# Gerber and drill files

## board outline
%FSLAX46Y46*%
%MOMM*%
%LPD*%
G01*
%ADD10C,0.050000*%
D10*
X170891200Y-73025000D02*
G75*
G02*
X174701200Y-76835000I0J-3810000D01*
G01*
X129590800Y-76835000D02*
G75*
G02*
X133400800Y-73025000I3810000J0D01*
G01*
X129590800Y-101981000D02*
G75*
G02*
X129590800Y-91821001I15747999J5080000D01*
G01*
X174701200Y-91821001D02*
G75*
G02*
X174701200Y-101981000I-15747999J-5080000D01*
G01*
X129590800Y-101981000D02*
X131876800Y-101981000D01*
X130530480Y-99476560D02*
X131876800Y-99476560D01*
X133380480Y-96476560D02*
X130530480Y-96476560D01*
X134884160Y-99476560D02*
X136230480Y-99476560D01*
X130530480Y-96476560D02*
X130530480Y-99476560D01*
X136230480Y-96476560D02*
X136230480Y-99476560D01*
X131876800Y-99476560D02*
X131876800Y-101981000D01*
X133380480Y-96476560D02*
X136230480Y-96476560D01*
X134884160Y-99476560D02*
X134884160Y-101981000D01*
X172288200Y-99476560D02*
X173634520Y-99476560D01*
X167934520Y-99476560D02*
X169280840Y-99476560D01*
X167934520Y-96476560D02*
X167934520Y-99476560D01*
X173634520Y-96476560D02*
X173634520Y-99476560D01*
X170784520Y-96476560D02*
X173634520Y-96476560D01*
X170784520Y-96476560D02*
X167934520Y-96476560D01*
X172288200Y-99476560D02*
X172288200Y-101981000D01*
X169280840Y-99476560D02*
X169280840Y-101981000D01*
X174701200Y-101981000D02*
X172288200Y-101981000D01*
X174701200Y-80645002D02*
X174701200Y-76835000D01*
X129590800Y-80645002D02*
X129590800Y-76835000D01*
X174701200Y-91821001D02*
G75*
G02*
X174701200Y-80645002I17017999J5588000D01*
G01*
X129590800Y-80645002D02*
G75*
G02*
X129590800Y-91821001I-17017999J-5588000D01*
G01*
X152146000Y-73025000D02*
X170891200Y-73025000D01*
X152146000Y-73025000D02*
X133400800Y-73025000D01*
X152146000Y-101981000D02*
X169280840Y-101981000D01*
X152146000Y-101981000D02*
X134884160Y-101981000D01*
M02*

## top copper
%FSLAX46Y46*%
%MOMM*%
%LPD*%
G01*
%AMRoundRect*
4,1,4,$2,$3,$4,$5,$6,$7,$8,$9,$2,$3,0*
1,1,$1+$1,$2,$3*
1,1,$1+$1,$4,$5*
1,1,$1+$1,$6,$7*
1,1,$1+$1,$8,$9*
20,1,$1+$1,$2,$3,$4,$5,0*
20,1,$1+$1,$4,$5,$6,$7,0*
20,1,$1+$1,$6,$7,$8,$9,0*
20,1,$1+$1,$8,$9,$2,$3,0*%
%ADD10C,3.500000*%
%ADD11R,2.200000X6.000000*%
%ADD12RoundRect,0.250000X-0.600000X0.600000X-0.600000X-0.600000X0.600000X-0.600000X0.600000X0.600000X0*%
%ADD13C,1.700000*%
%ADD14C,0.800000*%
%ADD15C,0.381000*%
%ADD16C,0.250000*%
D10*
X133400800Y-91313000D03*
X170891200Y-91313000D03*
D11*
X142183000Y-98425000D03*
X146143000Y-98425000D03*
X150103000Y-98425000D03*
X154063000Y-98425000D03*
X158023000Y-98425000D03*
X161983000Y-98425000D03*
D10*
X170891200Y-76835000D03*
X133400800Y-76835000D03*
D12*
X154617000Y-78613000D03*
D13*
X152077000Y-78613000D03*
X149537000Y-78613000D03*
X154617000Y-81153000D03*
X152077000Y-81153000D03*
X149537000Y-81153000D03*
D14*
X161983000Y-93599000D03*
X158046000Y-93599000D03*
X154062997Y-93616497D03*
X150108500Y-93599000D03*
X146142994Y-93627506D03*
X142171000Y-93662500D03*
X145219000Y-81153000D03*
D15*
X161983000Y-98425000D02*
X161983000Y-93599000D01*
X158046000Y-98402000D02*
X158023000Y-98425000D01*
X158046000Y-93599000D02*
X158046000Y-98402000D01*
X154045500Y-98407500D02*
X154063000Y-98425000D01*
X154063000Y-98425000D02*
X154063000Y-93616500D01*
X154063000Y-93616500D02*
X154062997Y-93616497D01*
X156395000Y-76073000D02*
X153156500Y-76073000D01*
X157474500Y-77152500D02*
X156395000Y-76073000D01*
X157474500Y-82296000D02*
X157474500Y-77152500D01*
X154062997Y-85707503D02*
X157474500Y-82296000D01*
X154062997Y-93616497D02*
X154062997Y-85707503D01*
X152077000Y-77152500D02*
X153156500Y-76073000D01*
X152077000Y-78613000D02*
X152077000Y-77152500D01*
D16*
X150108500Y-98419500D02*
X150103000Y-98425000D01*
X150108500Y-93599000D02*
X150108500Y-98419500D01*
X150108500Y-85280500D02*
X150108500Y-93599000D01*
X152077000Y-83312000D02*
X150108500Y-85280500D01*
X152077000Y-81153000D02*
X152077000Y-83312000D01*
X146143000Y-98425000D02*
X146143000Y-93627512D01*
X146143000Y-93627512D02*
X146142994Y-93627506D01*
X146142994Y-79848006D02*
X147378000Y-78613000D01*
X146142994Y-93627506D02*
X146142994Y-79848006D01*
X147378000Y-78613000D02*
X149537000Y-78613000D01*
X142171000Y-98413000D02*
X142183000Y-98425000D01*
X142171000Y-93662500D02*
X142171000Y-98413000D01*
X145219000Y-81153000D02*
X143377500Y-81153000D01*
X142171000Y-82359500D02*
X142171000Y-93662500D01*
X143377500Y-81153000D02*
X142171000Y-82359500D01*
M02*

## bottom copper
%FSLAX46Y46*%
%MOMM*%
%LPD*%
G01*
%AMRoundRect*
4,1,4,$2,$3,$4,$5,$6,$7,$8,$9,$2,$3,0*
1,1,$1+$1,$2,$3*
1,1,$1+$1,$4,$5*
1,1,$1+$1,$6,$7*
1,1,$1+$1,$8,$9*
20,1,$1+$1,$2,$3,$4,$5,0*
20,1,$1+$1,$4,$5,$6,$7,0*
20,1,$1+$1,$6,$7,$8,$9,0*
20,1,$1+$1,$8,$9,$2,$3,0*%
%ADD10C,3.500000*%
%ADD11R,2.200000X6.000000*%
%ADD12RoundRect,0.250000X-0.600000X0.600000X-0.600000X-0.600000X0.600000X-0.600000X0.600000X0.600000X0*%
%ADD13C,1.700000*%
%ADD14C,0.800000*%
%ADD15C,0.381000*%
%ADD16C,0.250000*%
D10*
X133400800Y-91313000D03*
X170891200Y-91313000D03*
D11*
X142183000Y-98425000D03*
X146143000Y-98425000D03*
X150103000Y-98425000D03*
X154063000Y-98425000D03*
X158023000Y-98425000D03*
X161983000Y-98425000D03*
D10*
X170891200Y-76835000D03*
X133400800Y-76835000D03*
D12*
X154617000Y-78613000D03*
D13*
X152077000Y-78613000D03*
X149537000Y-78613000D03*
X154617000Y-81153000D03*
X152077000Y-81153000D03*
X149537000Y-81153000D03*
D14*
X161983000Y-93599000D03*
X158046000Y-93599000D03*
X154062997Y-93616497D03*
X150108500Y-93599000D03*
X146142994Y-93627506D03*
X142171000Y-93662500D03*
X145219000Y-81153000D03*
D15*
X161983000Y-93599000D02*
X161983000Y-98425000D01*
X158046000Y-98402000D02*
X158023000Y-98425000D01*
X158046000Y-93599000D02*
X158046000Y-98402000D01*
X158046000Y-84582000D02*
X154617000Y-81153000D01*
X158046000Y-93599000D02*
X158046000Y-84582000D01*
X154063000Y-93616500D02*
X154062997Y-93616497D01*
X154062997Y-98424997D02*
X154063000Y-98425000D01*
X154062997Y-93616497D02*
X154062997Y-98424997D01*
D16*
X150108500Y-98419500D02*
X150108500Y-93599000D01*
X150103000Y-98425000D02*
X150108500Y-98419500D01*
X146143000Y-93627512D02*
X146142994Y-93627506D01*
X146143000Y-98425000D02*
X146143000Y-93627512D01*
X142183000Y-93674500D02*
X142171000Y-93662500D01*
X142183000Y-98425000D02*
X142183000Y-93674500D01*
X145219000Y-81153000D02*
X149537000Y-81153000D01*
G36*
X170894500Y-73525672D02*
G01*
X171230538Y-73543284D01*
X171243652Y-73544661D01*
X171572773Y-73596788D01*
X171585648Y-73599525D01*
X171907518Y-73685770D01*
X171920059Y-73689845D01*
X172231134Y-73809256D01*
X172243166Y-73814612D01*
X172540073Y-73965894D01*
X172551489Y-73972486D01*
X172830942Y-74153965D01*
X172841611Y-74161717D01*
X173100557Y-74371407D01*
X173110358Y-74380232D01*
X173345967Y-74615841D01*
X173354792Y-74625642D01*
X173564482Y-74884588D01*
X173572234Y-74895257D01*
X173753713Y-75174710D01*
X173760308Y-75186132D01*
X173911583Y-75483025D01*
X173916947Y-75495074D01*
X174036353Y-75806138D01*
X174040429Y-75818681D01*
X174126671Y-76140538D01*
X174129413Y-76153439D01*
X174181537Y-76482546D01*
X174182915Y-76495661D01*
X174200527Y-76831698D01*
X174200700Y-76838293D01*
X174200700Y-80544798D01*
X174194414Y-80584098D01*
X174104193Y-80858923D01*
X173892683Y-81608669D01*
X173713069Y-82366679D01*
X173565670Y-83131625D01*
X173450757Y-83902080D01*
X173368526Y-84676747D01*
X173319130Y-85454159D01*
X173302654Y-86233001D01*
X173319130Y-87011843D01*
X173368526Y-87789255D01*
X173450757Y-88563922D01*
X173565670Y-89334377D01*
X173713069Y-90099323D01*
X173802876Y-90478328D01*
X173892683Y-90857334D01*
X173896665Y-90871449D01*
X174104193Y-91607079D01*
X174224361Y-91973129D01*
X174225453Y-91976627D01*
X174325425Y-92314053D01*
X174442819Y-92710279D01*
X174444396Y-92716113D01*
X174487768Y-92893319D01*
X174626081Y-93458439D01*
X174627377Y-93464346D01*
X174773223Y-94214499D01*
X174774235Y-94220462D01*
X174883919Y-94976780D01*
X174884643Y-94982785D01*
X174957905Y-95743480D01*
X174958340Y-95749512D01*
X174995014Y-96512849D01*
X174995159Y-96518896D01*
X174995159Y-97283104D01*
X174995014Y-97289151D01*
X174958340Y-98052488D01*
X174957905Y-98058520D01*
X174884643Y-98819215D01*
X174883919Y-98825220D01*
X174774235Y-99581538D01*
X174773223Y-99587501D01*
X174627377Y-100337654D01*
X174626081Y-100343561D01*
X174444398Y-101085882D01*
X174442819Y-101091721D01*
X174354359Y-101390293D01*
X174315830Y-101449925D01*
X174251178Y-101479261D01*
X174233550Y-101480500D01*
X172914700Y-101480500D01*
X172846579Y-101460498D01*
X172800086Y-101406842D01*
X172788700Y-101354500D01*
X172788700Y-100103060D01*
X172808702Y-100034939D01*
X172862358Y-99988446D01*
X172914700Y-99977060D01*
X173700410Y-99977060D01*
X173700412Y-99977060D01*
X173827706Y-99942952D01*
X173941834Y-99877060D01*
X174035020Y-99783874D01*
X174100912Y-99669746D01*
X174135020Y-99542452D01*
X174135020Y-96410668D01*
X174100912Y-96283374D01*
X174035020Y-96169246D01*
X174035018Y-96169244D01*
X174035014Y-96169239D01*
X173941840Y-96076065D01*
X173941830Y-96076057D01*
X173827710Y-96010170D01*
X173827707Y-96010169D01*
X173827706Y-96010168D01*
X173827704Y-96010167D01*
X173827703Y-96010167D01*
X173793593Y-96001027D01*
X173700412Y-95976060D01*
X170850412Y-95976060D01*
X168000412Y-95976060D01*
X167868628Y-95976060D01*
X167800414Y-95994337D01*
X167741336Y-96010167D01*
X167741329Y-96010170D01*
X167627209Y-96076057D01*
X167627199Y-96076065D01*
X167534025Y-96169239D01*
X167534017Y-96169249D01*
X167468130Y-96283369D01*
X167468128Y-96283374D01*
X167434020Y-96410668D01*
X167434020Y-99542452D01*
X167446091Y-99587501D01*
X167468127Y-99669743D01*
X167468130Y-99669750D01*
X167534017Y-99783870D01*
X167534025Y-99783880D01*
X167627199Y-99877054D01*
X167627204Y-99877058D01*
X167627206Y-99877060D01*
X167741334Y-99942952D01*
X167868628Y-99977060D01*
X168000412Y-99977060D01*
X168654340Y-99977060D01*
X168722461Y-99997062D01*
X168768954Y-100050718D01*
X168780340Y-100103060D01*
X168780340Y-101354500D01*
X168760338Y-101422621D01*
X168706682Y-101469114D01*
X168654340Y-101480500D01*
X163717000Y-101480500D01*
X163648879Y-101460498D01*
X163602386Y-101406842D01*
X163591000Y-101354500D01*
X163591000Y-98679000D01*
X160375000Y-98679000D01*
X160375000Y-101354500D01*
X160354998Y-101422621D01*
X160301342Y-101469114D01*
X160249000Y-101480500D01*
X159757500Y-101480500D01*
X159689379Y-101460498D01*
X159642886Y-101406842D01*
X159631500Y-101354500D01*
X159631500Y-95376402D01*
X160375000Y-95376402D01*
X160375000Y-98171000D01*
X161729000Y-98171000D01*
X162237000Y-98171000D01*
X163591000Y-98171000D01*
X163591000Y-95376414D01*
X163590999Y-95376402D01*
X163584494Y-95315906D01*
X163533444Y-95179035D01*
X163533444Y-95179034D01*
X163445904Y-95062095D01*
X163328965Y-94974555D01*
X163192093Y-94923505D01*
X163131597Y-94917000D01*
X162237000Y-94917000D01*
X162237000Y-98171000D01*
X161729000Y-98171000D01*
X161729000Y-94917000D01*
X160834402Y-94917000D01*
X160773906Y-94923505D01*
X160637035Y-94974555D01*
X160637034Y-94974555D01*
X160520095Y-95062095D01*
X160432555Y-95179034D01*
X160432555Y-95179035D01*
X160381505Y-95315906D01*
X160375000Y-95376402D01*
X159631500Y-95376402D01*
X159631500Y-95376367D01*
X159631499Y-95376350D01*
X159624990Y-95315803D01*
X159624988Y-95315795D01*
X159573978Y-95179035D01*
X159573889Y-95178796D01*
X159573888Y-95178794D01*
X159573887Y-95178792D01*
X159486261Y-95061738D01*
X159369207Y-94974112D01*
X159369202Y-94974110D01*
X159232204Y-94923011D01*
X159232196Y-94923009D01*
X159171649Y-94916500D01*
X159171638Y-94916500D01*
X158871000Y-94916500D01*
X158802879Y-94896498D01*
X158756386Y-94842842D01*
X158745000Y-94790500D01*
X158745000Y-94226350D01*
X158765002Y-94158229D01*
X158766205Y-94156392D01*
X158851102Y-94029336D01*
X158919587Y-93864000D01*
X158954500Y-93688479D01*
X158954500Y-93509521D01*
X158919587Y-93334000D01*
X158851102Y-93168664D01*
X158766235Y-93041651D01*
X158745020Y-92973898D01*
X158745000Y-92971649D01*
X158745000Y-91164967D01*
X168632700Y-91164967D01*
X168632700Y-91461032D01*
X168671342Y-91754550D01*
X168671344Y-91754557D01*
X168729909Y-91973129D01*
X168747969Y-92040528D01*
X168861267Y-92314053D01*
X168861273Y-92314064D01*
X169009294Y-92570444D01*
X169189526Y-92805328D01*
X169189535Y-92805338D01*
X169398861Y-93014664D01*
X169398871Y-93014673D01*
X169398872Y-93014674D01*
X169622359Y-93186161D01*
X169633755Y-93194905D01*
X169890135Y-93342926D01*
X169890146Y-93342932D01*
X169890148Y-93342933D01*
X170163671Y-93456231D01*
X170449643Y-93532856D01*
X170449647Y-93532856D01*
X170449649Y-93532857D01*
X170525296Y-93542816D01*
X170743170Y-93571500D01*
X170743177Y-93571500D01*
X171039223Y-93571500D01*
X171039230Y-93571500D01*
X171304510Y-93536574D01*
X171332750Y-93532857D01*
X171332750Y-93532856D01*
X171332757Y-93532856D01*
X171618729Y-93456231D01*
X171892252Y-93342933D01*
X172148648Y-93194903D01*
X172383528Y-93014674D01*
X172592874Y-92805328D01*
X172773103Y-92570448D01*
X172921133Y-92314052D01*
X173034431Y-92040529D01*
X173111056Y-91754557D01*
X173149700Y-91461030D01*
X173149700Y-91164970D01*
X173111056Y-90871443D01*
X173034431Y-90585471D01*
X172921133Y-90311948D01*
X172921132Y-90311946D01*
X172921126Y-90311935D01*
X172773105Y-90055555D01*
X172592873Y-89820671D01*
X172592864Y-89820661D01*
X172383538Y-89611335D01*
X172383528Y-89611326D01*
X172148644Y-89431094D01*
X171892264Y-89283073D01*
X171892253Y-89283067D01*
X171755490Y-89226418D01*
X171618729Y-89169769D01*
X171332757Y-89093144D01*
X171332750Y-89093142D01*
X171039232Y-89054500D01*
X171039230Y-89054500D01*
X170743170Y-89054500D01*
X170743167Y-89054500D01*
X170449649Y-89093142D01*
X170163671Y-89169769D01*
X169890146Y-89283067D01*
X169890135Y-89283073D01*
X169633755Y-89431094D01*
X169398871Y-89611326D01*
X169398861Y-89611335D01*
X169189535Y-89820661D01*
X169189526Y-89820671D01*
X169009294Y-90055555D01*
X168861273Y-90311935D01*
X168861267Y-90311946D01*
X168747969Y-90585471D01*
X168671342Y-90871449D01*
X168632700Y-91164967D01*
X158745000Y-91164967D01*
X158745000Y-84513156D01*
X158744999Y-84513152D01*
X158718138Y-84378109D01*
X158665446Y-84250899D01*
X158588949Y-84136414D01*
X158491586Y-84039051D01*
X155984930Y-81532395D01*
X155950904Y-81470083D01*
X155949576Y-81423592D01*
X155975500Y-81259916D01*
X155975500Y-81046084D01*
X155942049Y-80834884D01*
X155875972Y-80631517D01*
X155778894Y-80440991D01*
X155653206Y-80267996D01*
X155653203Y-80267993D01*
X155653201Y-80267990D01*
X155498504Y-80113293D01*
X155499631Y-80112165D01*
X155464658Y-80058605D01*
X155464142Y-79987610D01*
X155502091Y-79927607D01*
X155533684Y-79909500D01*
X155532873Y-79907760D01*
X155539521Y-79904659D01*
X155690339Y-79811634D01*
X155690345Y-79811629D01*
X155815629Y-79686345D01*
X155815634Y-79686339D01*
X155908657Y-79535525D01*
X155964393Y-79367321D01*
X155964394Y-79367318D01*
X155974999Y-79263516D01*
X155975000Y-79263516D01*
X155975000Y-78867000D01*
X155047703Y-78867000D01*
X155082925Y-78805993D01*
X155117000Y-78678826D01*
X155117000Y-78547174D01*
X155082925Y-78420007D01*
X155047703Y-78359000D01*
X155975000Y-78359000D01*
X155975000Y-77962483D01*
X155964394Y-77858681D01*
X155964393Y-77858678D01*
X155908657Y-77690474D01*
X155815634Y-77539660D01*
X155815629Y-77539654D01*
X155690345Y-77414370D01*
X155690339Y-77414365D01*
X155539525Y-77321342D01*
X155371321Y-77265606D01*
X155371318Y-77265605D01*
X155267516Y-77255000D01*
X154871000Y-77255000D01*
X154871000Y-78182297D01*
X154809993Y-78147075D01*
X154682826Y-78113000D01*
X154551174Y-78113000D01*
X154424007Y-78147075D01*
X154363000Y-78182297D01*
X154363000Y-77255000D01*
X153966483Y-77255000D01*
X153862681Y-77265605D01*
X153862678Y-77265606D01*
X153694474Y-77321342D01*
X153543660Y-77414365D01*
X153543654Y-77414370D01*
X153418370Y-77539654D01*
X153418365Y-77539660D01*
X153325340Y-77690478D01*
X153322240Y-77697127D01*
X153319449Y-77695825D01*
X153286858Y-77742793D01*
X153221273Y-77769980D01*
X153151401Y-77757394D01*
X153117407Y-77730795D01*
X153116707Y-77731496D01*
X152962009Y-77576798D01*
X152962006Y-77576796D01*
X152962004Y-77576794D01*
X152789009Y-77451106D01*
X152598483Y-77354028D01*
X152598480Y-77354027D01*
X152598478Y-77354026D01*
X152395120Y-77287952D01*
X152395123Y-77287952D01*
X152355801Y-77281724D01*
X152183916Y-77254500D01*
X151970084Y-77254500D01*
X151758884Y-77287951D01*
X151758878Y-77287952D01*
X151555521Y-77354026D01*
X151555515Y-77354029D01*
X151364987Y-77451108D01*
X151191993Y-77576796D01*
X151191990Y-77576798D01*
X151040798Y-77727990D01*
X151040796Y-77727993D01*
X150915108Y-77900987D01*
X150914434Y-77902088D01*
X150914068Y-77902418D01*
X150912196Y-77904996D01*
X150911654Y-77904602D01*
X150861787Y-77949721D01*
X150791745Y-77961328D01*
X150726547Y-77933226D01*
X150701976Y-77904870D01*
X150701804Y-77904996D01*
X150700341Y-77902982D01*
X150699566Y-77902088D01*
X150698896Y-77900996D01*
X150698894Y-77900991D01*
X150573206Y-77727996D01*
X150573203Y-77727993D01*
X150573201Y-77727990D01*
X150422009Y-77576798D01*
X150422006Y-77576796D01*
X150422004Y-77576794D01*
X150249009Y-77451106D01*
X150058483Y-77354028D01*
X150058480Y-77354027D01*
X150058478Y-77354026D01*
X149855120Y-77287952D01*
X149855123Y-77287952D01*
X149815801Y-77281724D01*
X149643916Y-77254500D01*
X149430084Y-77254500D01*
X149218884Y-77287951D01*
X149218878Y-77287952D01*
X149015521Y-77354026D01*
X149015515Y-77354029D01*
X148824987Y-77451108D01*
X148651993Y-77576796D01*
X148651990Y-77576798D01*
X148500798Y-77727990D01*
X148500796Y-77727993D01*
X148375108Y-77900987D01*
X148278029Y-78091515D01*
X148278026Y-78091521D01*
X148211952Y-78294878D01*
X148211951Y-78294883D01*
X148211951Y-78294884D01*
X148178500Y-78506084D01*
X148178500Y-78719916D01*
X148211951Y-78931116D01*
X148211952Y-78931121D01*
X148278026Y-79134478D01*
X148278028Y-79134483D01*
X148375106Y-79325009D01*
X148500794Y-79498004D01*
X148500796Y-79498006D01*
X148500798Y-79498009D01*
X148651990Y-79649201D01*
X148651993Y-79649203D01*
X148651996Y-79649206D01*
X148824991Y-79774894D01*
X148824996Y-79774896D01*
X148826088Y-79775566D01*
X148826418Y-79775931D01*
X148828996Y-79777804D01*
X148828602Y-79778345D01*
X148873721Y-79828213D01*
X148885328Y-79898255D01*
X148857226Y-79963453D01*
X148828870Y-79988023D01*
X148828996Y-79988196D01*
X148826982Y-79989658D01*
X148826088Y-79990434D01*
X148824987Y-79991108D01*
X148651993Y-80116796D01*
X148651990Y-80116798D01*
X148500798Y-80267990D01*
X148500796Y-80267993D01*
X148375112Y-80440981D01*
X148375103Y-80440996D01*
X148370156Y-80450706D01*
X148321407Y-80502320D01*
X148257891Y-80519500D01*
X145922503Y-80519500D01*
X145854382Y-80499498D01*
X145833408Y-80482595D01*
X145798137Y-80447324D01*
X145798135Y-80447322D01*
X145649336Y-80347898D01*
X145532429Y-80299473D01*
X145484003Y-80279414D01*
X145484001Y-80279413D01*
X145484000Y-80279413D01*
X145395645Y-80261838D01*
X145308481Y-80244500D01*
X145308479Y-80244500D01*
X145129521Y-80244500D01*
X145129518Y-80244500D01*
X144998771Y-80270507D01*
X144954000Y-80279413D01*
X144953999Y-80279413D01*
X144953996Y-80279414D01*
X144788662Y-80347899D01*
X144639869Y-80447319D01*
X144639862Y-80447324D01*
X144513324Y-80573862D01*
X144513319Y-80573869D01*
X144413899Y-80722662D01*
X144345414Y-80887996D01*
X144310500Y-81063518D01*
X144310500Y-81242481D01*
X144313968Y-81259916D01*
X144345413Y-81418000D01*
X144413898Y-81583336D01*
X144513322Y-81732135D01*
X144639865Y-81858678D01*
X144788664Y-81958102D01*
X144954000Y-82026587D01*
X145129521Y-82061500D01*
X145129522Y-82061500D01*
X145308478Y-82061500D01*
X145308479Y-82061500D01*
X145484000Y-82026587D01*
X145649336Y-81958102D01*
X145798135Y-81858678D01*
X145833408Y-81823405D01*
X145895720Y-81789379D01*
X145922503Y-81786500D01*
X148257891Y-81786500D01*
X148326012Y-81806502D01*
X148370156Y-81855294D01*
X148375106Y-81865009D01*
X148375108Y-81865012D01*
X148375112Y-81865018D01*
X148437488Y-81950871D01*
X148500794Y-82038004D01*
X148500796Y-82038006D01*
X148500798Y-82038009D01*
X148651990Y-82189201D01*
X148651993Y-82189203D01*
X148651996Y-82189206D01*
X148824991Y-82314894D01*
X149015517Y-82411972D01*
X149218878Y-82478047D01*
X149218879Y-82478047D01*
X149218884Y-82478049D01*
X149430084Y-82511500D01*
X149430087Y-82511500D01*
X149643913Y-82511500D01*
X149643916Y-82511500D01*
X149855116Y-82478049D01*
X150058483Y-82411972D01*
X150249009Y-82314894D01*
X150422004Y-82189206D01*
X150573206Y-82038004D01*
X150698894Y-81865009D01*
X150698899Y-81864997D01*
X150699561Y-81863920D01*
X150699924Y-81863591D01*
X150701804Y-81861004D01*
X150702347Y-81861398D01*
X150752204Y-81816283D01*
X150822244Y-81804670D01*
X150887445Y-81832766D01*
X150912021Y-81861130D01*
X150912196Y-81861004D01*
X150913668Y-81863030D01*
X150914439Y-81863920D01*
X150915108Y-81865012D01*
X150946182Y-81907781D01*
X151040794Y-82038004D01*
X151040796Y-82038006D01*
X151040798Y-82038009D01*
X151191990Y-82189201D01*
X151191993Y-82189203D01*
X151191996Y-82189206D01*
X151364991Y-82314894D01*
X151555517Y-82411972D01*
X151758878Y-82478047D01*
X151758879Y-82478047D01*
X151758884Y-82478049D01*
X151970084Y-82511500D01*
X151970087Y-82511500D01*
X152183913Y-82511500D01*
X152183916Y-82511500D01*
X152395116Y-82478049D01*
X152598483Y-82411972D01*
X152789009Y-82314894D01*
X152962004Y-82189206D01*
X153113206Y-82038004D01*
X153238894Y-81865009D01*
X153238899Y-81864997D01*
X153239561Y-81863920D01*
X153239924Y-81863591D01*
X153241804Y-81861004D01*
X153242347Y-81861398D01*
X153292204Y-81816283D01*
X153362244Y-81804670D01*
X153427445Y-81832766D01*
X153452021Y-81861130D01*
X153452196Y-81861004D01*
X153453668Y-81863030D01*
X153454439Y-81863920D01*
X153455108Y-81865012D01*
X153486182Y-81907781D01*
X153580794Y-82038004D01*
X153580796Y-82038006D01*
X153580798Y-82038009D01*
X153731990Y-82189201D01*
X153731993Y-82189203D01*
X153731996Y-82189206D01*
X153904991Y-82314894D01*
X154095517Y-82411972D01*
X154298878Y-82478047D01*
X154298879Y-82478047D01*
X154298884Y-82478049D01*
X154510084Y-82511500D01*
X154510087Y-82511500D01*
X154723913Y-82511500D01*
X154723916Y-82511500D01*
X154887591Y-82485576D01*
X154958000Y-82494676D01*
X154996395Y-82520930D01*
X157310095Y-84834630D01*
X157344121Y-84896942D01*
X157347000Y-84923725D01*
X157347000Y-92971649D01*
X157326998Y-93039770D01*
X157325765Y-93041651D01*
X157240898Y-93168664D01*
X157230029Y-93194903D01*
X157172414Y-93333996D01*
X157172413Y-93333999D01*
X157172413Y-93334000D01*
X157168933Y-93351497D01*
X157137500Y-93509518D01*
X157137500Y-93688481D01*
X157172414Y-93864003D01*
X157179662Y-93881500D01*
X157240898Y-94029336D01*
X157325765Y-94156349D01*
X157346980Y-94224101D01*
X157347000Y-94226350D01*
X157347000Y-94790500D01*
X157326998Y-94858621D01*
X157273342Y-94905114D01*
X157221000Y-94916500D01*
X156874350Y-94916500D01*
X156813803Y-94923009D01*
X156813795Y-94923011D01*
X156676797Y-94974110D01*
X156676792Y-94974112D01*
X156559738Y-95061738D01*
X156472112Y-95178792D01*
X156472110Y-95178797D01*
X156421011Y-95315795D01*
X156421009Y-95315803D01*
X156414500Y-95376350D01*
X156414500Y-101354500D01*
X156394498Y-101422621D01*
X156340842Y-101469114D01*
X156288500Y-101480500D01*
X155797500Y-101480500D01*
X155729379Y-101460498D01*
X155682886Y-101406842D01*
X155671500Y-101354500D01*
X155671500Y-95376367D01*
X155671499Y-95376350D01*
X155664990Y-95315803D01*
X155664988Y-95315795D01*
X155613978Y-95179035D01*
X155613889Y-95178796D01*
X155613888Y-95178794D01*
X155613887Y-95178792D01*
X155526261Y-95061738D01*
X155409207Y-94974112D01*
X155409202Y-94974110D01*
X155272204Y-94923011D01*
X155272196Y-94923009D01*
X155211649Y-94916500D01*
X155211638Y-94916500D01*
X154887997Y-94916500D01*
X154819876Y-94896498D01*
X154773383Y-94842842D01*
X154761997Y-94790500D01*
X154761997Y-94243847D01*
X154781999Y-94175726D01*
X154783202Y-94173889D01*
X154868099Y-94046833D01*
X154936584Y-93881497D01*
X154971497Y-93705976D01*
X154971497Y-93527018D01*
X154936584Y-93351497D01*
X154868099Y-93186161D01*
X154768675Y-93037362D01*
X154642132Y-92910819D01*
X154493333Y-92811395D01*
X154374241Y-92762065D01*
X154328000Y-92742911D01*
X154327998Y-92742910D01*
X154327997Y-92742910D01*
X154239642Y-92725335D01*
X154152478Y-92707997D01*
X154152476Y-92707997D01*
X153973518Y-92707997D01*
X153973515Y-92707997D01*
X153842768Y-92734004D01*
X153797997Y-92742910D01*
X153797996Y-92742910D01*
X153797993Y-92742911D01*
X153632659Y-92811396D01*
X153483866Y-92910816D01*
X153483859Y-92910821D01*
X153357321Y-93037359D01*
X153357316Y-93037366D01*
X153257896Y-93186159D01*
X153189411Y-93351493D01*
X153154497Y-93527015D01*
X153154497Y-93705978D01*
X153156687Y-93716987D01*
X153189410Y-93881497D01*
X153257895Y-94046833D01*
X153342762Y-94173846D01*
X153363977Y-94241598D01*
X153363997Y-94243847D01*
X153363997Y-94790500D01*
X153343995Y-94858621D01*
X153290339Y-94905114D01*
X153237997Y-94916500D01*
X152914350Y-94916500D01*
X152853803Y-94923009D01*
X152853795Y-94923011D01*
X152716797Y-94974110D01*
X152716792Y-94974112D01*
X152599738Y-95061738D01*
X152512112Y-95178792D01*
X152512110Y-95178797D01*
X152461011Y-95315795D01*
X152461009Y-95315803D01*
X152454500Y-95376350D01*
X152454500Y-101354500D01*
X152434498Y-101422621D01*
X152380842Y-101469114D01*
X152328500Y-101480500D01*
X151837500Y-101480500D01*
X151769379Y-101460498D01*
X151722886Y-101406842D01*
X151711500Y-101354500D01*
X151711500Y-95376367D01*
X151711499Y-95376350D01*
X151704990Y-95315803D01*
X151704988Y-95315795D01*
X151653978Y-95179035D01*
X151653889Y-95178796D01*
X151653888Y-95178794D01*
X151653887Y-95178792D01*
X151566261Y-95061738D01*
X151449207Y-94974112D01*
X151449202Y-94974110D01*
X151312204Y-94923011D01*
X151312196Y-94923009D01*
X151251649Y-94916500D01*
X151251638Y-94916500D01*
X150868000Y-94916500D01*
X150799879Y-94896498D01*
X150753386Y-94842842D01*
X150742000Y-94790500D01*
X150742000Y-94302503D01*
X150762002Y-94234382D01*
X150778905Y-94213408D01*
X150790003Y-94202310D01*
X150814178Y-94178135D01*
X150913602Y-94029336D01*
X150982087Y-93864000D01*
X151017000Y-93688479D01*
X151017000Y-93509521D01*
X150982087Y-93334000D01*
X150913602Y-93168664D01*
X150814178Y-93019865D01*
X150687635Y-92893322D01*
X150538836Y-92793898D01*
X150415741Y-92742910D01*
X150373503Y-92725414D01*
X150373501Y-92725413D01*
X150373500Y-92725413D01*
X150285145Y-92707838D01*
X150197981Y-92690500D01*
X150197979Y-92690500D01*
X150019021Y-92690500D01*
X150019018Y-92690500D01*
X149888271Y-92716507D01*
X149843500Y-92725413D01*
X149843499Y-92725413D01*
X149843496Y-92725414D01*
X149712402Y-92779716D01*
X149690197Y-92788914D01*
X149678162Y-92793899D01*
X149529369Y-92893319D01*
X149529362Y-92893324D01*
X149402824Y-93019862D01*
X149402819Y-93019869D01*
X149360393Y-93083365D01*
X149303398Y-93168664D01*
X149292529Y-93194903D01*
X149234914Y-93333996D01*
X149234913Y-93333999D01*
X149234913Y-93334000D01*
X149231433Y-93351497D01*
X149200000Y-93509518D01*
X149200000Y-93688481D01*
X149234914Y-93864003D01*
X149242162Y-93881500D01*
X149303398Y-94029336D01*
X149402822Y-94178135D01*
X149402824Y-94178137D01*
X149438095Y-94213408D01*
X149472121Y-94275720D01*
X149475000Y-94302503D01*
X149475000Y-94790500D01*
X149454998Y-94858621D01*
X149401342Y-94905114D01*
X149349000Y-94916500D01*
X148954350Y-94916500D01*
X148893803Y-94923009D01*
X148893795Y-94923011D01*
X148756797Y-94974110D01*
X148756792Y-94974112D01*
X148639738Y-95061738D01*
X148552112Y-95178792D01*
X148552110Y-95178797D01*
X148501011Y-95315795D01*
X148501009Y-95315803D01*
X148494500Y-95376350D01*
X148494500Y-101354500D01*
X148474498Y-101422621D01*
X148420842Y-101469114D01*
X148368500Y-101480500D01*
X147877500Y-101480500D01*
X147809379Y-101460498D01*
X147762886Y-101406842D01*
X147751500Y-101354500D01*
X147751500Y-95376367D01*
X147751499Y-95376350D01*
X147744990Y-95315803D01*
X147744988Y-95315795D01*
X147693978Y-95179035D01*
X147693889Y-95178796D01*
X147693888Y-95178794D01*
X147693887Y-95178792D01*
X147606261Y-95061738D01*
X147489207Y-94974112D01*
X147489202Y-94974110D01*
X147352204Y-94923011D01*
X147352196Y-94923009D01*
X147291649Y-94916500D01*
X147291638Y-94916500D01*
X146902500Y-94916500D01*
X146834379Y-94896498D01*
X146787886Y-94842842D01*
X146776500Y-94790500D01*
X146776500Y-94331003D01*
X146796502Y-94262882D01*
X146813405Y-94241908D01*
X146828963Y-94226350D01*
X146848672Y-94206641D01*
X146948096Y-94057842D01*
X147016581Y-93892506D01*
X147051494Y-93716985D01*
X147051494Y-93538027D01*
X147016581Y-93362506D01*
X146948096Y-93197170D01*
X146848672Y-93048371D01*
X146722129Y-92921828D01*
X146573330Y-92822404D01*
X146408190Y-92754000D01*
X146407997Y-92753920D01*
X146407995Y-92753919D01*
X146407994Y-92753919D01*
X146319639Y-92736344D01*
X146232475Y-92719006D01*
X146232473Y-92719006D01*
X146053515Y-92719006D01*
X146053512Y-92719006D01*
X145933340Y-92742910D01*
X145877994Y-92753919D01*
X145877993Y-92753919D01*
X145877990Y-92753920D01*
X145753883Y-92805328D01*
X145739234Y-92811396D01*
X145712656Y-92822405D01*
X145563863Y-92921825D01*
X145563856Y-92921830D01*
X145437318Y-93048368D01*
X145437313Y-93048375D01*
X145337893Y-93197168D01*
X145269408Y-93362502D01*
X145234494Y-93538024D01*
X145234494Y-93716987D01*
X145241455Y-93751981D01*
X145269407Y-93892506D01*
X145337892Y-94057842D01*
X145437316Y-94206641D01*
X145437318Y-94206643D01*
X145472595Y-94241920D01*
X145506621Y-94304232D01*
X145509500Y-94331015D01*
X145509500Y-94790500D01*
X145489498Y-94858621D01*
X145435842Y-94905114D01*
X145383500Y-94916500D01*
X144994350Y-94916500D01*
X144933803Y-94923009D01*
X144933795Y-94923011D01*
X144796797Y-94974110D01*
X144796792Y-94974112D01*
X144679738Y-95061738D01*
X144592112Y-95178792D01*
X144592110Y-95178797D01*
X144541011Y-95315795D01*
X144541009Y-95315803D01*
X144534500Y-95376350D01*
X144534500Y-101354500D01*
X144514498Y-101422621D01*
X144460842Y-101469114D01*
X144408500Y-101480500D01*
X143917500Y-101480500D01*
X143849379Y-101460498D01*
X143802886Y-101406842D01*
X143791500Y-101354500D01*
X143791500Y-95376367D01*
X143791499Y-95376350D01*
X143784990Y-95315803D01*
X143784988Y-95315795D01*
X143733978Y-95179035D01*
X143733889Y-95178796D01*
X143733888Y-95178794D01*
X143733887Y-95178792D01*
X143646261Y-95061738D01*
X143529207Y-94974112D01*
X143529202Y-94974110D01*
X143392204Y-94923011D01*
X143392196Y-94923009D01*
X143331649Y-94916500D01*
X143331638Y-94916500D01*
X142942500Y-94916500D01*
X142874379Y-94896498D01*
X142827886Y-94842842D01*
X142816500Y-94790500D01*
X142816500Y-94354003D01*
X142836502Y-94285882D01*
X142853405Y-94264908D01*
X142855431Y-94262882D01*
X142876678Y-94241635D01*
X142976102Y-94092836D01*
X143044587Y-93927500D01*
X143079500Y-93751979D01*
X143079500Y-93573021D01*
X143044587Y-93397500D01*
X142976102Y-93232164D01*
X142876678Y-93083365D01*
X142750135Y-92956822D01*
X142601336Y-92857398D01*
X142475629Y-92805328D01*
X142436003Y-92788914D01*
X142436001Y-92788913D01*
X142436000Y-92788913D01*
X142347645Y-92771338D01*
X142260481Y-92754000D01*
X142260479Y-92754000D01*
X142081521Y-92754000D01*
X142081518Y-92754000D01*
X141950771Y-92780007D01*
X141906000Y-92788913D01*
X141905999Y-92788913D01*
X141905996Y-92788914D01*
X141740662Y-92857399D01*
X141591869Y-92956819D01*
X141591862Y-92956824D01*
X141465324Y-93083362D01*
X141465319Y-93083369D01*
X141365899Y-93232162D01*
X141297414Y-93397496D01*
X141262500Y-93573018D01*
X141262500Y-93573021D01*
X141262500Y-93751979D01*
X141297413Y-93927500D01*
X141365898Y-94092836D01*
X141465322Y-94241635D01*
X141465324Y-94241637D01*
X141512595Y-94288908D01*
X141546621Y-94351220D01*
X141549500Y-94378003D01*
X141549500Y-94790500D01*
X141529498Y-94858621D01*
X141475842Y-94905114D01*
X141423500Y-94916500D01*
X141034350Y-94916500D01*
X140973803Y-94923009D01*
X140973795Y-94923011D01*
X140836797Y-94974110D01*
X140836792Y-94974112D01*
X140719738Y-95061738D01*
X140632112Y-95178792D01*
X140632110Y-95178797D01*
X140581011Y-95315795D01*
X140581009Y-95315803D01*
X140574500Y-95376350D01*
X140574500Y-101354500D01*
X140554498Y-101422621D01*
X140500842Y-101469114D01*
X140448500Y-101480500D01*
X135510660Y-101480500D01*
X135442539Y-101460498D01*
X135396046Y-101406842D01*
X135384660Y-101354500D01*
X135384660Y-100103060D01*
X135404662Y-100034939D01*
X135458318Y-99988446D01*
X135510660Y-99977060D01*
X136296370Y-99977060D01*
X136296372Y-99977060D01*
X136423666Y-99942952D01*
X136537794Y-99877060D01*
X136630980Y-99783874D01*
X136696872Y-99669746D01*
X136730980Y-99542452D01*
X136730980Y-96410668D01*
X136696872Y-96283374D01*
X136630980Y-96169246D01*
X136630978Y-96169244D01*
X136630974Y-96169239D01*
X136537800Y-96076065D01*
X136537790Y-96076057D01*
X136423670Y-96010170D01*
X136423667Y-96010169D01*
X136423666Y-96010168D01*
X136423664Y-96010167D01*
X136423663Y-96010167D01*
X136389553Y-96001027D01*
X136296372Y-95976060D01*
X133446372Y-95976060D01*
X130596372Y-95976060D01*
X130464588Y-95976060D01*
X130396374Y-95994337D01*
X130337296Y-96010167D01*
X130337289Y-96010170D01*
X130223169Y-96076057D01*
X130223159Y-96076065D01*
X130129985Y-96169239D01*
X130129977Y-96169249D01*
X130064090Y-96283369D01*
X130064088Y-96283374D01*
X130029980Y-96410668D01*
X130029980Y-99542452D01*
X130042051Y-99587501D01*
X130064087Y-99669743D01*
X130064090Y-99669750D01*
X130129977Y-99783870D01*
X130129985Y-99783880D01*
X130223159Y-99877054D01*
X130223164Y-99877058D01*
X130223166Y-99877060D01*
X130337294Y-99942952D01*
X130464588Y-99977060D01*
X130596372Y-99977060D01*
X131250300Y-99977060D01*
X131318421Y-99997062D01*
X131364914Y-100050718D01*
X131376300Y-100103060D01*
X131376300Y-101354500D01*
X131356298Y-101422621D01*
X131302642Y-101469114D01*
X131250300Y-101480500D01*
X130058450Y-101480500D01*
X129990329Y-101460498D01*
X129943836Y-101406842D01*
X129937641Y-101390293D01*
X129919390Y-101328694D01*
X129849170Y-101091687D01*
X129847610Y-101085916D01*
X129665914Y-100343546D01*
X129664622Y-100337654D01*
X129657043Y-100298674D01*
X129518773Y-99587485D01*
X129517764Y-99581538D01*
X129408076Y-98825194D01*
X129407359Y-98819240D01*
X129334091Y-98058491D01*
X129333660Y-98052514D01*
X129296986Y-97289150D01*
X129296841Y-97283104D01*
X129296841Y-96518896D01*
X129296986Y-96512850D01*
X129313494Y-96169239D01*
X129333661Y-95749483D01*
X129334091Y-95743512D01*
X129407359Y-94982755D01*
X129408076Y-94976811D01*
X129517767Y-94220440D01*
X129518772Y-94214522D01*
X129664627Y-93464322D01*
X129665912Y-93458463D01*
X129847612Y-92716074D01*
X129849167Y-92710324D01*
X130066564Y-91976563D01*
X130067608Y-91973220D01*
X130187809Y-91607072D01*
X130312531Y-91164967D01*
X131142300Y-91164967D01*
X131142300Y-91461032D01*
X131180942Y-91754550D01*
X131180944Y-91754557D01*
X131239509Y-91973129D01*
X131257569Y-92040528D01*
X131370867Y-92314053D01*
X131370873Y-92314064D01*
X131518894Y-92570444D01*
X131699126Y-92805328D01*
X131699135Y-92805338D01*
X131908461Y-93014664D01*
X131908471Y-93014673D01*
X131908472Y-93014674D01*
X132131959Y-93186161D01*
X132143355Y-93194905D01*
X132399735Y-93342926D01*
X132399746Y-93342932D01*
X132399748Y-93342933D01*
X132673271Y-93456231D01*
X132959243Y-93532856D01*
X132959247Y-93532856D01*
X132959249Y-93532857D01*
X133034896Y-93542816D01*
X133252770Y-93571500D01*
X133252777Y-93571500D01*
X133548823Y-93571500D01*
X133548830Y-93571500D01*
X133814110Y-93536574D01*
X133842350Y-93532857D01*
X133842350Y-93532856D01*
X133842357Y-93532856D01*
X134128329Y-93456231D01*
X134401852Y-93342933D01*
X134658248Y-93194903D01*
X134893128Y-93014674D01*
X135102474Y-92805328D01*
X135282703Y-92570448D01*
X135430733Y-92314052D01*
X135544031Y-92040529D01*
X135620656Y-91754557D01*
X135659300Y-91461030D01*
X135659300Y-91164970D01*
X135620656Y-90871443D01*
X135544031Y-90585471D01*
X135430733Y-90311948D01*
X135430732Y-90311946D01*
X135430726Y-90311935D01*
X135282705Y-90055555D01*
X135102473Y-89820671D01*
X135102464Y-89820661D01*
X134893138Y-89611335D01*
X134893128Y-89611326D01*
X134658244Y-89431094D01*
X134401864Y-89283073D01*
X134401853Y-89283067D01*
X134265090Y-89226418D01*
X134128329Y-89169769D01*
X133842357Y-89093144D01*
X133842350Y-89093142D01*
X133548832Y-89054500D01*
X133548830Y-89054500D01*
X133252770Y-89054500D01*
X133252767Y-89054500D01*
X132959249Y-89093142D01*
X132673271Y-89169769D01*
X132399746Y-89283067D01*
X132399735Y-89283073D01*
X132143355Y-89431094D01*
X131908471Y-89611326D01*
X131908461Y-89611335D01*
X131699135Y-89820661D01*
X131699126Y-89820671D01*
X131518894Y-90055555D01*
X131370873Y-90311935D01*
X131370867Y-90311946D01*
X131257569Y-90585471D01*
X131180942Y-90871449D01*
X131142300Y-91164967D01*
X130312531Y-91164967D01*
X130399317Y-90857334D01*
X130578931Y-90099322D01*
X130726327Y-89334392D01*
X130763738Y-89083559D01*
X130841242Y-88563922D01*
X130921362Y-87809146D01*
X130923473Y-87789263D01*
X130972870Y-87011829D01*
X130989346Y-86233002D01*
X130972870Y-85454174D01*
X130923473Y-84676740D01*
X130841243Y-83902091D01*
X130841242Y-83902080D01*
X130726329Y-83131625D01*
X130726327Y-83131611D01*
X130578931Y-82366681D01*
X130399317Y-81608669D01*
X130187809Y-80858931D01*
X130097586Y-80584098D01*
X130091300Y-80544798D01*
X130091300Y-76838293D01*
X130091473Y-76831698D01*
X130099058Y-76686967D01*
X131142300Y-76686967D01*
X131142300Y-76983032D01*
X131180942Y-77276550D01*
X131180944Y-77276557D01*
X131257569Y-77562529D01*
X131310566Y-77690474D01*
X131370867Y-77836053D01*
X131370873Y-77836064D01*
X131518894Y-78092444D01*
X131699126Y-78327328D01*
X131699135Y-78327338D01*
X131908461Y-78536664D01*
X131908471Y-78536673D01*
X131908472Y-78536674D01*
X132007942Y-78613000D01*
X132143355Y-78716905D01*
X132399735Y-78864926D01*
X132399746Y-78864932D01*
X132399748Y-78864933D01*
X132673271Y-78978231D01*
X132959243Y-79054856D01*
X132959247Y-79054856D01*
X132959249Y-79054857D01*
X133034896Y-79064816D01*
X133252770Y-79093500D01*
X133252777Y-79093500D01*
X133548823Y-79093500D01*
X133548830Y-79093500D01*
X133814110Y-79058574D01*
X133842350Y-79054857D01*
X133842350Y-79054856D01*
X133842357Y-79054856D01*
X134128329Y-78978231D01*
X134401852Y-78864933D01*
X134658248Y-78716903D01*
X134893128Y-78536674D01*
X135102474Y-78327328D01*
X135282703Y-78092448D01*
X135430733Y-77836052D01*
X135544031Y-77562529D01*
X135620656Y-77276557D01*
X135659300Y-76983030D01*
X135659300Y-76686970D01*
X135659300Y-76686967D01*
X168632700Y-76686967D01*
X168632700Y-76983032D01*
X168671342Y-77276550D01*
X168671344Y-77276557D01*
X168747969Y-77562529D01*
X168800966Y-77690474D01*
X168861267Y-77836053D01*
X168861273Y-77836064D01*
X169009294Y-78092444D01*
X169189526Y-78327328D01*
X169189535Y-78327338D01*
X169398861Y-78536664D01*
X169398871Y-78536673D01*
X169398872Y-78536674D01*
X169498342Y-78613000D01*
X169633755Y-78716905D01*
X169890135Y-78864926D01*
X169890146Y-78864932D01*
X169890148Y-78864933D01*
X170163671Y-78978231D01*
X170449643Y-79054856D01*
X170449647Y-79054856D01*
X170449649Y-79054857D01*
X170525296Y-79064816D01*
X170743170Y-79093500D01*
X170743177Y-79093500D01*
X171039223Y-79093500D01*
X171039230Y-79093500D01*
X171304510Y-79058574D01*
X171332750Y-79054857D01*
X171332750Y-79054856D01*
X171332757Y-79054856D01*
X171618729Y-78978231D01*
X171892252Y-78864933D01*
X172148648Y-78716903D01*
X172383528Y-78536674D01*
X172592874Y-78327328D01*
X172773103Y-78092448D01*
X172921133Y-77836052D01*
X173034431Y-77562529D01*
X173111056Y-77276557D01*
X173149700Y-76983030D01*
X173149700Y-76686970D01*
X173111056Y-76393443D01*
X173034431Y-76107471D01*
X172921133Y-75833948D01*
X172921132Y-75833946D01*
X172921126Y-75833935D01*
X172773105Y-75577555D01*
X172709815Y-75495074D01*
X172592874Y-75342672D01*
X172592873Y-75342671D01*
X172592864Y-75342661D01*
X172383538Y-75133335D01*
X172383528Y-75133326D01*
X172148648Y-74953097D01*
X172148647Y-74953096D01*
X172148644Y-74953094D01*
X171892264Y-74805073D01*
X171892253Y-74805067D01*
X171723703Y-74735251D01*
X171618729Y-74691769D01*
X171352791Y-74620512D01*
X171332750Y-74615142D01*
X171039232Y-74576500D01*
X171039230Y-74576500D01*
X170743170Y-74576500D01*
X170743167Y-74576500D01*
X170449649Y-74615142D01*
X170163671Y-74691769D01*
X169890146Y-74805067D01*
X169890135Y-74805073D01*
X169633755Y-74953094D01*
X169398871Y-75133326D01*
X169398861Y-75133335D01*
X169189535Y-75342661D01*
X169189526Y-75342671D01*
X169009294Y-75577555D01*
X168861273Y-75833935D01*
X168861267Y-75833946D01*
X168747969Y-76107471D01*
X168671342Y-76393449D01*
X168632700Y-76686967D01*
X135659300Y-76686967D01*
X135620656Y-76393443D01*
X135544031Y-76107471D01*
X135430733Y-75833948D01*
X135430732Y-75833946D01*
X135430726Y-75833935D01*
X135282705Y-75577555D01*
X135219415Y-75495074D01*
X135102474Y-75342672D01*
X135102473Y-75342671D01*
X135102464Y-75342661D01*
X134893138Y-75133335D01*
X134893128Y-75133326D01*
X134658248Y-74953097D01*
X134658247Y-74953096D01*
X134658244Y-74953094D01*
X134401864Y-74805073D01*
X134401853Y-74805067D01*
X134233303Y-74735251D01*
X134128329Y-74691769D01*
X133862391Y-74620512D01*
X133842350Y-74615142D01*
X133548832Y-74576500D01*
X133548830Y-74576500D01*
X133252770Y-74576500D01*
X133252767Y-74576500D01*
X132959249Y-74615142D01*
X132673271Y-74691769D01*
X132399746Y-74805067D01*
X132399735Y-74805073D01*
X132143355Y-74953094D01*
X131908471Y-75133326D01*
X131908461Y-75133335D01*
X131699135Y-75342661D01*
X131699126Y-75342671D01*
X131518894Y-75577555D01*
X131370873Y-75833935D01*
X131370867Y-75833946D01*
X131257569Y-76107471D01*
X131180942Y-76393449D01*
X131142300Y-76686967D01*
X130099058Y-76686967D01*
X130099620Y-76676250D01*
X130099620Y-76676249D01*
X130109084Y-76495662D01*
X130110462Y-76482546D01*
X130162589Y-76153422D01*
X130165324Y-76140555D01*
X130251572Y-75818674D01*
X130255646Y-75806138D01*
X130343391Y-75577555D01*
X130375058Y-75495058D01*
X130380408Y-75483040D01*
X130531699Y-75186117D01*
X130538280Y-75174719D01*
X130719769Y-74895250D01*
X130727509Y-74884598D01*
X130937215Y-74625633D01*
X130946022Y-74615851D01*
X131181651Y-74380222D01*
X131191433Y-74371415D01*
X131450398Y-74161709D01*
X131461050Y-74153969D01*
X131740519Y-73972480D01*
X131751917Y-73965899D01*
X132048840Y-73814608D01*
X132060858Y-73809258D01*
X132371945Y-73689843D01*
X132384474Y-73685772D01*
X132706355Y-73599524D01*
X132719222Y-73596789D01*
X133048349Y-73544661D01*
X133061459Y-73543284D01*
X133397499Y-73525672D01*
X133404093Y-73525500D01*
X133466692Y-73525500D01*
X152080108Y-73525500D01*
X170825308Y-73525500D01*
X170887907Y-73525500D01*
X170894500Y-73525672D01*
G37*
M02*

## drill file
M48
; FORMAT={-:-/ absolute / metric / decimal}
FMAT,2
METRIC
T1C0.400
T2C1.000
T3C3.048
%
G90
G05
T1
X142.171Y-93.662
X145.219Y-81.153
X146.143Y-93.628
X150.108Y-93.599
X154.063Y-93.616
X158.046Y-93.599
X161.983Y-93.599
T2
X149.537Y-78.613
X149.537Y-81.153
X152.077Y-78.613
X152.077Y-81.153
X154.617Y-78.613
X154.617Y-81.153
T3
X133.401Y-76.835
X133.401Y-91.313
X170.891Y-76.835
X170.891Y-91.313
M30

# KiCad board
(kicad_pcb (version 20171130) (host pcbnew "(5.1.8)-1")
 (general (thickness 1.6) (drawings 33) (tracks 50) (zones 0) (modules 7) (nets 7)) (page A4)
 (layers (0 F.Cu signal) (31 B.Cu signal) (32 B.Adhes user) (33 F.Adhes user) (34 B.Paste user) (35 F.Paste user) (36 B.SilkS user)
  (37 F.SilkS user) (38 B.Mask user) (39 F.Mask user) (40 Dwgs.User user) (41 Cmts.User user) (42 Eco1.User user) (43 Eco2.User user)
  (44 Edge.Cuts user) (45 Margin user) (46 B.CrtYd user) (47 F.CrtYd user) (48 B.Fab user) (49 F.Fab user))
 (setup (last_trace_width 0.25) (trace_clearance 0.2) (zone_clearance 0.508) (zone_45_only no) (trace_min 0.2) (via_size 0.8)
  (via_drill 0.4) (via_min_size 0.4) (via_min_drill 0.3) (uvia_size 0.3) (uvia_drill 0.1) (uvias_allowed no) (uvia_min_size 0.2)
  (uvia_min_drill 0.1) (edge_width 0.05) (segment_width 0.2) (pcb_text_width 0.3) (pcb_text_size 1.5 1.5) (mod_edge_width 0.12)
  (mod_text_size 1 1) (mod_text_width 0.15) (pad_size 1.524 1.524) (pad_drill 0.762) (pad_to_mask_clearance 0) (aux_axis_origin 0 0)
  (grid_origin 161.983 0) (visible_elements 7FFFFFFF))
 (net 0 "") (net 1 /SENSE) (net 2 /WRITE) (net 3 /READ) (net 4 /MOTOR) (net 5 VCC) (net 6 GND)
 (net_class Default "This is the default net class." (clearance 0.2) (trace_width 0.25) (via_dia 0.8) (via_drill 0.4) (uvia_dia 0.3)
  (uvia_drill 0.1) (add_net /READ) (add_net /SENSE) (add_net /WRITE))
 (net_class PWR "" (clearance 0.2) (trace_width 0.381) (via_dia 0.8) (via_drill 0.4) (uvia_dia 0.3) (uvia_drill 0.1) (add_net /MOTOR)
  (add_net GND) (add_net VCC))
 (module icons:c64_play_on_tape (layer F.Cu) (at 152.0444 88.9508)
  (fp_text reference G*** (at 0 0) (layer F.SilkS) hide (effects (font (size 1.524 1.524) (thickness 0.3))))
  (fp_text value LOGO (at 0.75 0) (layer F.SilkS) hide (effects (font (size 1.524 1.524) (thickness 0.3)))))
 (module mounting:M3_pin (layer F.Cu) (at 133.4008 91.313)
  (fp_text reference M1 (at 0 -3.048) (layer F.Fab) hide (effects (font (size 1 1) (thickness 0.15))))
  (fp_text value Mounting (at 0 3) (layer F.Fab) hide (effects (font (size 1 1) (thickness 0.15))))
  (pad 1 thru_hole circle (at 0 0) (size 3.5 3.5) (drill 3.048) (layers *.Cu *.Mask) (solder_mask_margin 0.8)))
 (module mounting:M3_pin (layer F.Cu) (at 170.8912 91.313)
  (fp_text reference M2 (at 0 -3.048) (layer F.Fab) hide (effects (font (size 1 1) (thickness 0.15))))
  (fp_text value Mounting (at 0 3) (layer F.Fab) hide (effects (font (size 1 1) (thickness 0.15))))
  (pad 1 thru_hole circle (at 0 0) (size 3.5 3.5) (drill 3.048) (layers *.Cu *.Mask) (solder_mask_margin 0.8)))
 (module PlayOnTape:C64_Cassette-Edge (layer F.Cu) (at 173.863 98.425)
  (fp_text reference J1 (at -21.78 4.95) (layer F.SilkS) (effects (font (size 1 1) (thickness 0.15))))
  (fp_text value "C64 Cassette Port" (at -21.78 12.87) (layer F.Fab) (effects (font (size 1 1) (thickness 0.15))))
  (pad F smd rect (at -31.68 0) (size 2.2 6) (layers B.Cu B.Paste B.Mask) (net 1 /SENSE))
  (pad E smd rect (at -27.72 0) (size 2.2 6) (layers B.Cu B.Paste B.Mask) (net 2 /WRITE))
  (pad D smd rect (at -23.76 0) (size 2.2 6) (layers B.Cu B.Paste B.Mask) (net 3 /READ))
  (pad 6 smd rect (at -31.68 0) (size 2.2 6) (layers F.Cu F.Paste F.Mask) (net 1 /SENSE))
  (pad 5 smd rect (at -27.72 0) (size 2.2 6) (layers F.Cu F.Paste F.Mask) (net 2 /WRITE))
  (pad 4 smd rect (at -23.76 0) (size 2.2 6) (layers F.Cu F.Paste F.Mask) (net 3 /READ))
  (pad C smd rect (at -19.8 0) (size 2.2 6) (layers B.Cu B.Paste B.Mask) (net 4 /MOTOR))
  (pad B smd rect (at -15.84 0) (size 2.2 6) (layers B.Cu B.Paste B.Mask) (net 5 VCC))
  (pad A smd rect (at -11.88 0) (size 2.2 6) (layers B.Cu B.Paste B.Mask) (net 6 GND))
  (pad 3 smd rect (at -19.8 0) (size 2.2 6) (layers F.Cu F.Paste F.Mask) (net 4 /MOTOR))
  (pad 2 smd rect (at -15.84 0) (size 2.2 6) (layers F.Cu F.Paste F.Mask) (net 5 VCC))
  (pad 1 smd rect (at -11.88 0) (size 2.2 6) (layers F.Cu F.Paste F.Mask) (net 6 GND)))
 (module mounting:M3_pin (layer F.Cu) (at 170.8912 76.835)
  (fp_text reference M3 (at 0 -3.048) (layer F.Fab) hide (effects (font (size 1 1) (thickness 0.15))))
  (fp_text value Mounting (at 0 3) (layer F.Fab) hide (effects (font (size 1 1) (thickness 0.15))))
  (pad 1 thru_hole circle (at 0 0) (size 3.5 3.5) (drill 3.048) (layers *.Cu *.Mask) (solder_mask_margin 0.8)))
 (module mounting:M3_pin (layer F.Cu) (at 133.4008 76.835)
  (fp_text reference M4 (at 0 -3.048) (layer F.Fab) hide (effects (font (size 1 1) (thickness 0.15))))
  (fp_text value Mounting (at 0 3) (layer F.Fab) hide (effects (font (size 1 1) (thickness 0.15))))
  (pad 1 thru_hole circle (at 0 0) (size 3.5 3.5) (drill 3.048) (layers *.Cu *.Mask) (solder_mask_margin 0.8)))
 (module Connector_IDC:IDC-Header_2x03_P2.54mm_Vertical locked (layer F.Cu) (at 154.617 78.613 270)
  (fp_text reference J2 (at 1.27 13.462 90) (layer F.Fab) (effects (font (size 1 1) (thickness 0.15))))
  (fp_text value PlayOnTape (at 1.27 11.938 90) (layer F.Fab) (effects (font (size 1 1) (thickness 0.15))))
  (pad 1 thru_hole roundrect (at 0 0 270) (size 1.7 1.7) (drill 1) (layers *.Cu *.Mask) (roundrect_rratio 0.1470588235294118) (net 6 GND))
  (pad 3 thru_hole circle (at 0 2.54 270) (size 1.7 1.7) (drill 1) (layers *.Cu *.Mask) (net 4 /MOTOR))
  (pad 5 thru_hole circle (at 0 5.08 270) (size 1.7 1.7) (drill 1) (layers *.Cu *.Mask) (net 2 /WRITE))
  (pad 2 thru_hole circle (at 2.54 0 270) (size 1.7 1.7) (drill 1) (layers *.Cu *.Mask) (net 5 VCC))
  (pad 4 thru_hole circle (at 2.54 2.54 270) (size 1.7 1.7) (drill 1) (layers *.Cu *.Mask) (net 3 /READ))
  (pad 6 thru_hole circle (at 2.54 5.08 270) (size 1.7 1.7) (drill 1) (layers *.Cu *.Mask) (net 1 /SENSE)))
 (gr_arc (start 170.8912 76.835) (end 174.7012 76.835) (angle -90) (layer Edge.Cuts) (width 0.05))
 (gr_arc (start 133.4008 76.835) (end 133.4008 73.025) (angle -90) (layer Edge.Cuts) (width 0.05))
 (gr_arc (start 145.338799 96.901) (end 129.5908 91.821001) (angle -35.75739319) (layer Edge.Cuts) (width 0.05))
 (gr_arc (start 158.953201 96.901001) (end 174.7012 101.981) (angle -35.75739319) (layer Edge.Cuts) (width 0.05))
 (gr_line (start 129.5908 101.981) (end 131.8768 101.981) (layer Edge.Cuts) (width 0.05))
 (gr_line (start 130.53048 99.47656) (end 131.8768 99.47656) (layer Edge.Cuts) (width 0.05))
 (gr_line (start 133.38048 96.47656) (end 130.53048 96.47656) (layer Edge.Cuts) (width 0.05))
 (gr_line (start 134.88416 99.47656) (end 136.23048 99.47656) (layer Edge.Cuts) (width 0.05))
 (gr_line (start 130.53048 96.47656) (end 130.53048 99.47656) (layer Edge.Cuts) (width 0.05))
 (gr_line (start 136.23048 96.47656) (end 136.23048 99.47656) (layer Edge.Cuts) (width 0.05))
 (gr_line (start 131.8768 99.47656) (end 131.8768 101.981) (layer Edge.Cuts) (width 0.05))
 (gr_line (start 133.38048 96.47656) (end 136.23048 96.47656) (layer Edge.Cuts) (width 0.05))
 (gr_line (start 134.88416 99.47656) (end 134.88416 101.981) (layer Edge.Cuts) (width 0.05))
 (gr_line (start 172.2882 99.47656) (end 173.63452 99.47656) (layer Edge.Cuts) (width 0.05))
 (gr_line (start 167.93452 99.47656) (end 169.28084 99.47656) (layer Edge.Cuts) (width 0.05))
 (gr_line (start 167.93452 96.47656) (end 167.93452 99.47656) (layer Edge.Cuts) (width 0.05))
 (gr_line (start 173.63452 96.47656) (end 173.63452 99.47656) (layer Edge.Cuts) (width 0.05))
 (gr_line (start 170.78452 96.47656) (end 173.63452 96.47656) (layer Edge.Cuts) (width 0.05))
 (gr_line (start 170.78452 96.47656) (end 167.93452 96.47656) (layer Edge.Cuts) (width 0.05))
 (gr_line (start 172.2882 99.47656) (end 172.2882 101.981) (layer Edge.Cuts) (width 0.05))
 (gr_line (start 169.28084 99.47656) (end 169.28084 101.981) (layer Edge.Cuts) (width 0.05))
 (gr_line (start 174.7012 101.981) (end 172.2882 101.981) (layer Edge.Cuts) (width 0.05))
 (gr_line (start 174.7012 80.645002) (end 174.7012 76.835) (layer Edge.Cuts) (width 0.05))
 (gr_line (start 129.5908 80.645002) (end 129.5908 76.835) (layer Edge.Cuts) (width 0.05))
 (gr_arc (start 191.719199 86.233001) (end 174.7012 80.645002) (angle -36.3560376) (layer Edge.Cuts) (width 0.05))
 (gr_arc (start 112.572801 86.233002) (end 129.5908 91.821001) (angle -36.3560376) (layer Edge.Cuts) (width 0.05))
 (gr_line (start 152.146 73.025) (end 170.8912 73.025) (layer Edge.Cuts) (width 0.05))
 (gr_line (start 152.146 73.025) (end 133.4008 73.025) (layer Edge.Cuts) (width 0.05))
 (gr_line (start 152.146 101.981) (end 169.28084 101.981) (layer Edge.Cuts) (width 0.05))
 (gr_line (start 152.146 101.981) (end 134.88416 101.981) (layer Edge.Cuts) (width 0.05))
 (segment (start 161.983 98.425) (end 161.983 93.599) (width 0.381) (layer F.Cu) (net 6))
 (via (at 161.983 93.599) (size 0.8) (drill 0.4) (layers F.Cu B.Cu) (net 6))
 (segment (start 161.983 93.599) (end 161.983 98.425) (width 0.381) (layer B.Cu) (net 6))
 (via (at 158.046 93.599) (size 0.8) (drill 0.4) (layers F.Cu B.Cu) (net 5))
 (segment (start 158.046 98.402) (end 158.023 98.425) (width 0.381) (layer F.Cu) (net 5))
 (segment (start 158.046 93.599) (end 158.046 98.402) (width 0.381) (layer F.Cu) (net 5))
 (segment (start 158.046 98.402) (end 158.023 98.425) (width 0.381) (layer B.Cu) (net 5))
 (segment (start 158.046 93.599) (end 158.046 98.402) (width 0.381) (layer B.Cu) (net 5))
 (segment (start 158.046 84.582) (end 154.617 81.153) (width 0.381) (layer B.Cu) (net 5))
 (segment (start 158.046 93.599) (end 158.046 84.582) (width 0.381) (layer B.Cu) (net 5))
 (segment (start 154.0455 98.4075) (end 154.063 98.425) (width 0.381) (layer F.Cu) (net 4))
 (via (at 154.062997 93.616497) (size 0.8) (drill 0.4) (layers F.Cu B.Cu) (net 4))
 (segment (start 154.063 93.6165) (end 154.062997 93.616497) (width 0.381) (layer B.Cu) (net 4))
 (segment (start 154.063 98.425) (end 154.063 93.6165) (width 0.381) (layer F.Cu) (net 4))
 (segment (start 154.063 93.6165) (end 154.062997 93.616497) (width 0.381) (layer F.Cu) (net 4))
 (segment (start 154.062997 98.424997) (end 154.063 98.425) (width 0.381) (layer B.Cu) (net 4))
 (segment (start 154.062997 93.616497) (end 154.062997 98.424997) (width 0.381) (layer B.Cu) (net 4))
 (segment (start 156.395 76.073) (end 153.1565 76.073) (width 0.381) (layer F.Cu) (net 4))
 (segment (start 157.4745 77.1525) (end 156.395 76.073) (width 0.381) (layer F.Cu) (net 4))
 (segment (start 157.4745 82.296) (end 157.4745 77.1525) (width 0.381) (layer F.Cu) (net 4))
 (segment (start 154.062997 85.707503) (end 157.4745 82.296) (width 0.381) (layer F.Cu) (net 4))
 (segment (start 154.062997 93.616497) (end 154.062997 85.707503) (width 0.381) (layer F.Cu) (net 4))
 (segment (start 152.077 77.1525) (end 153.1565 76.073) (width 0.381) (layer F.Cu) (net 4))
 (segment (start 152.077 78.613) (end 152.077 77.1525) (width 0.381) (layer F.Cu) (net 4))
 (via (at 150.1085 93.599) (size 0.8) (drill 0.4) (layers F.Cu B.Cu) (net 3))
 (segment (start 150.1085 98.4195) (end 150.103 98.425) (width 0.25) (layer F.Cu) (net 3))
 (segment (start 150.1085 93.599) (end 150.1085 98.4195) (width 0.25) (layer F.Cu) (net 3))
 (segment (start 150.1085 98.4195) (end 150.1085 93.599) (width 0.25) (layer B.Cu) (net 3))
 (segment (start 150.103 98.425) (end 150.1085 98.4195) (width 0.25) (layer B.Cu) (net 3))
 (segment (start 150.1085 85.2805) (end 150.1085 93.599) (width 0.25) (layer F.Cu) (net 3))
 (segment (start 152.077 83.312) (end 150.1085 85.2805) (width 0.25) (layer F.Cu) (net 3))
 (segment (start 152.077 81.153) (end 152.077 83.312) (width 0.25) (layer F.Cu) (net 3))
 (via (at 146.142994 93.627506) (size 0.8) (drill 0.4) (layers F.Cu B.Cu) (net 2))
 (segment (start 146.143 98.425) (end 146.143 93.627512) (width 0.25) (layer F.Cu) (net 2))
 (segment (start 146.143 93.627512) (end 146.142994 93.627506) (width 0.25) (layer F.Cu) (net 2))
 (segment (start 146.143 93.627512) (end 146.142994 93.627506) (width 0.25) (layer B.Cu) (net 2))
 (segment (start 146.143 98.425) (end 146.143 93.627512) (width 0.25) (layer B.Cu) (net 2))
 (segment (start 146.142994 79.848006) (end 147.378 78.613) (width 0.25) (layer F.Cu) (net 2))
 (segment (start 146.142994 93.627506) (end 146.142994 79.848006) (width 0.25) (layer F.Cu) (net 2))
 (segment (start 147.378 78.613) (end 149.537 78.613) (width 0.25) (layer F.Cu) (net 2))
 (segment (start 142.183 93.6745) (end 142.171 93.6625) (width 0.25) (layer B.Cu) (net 1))
 (segment (start 142.183 98.425) (end 142.183 93.6745) (width 0.25) (layer B.Cu) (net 1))
 (via (at 142.171 93.6625) (size 0.8) (drill 0.4) (layers F.Cu B.Cu) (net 1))
 (segment (start 142.171 98.413) (end 142.183 98.425) (width 0.25) (layer F.Cu) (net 1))
 (segment (start 142.171 93.6625) (end 142.171 98.413) (width 0.25) (layer F.Cu) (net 1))
 (via (at 145.219 81.153) (size 0.8) (drill 0.4) (layers F.Cu B.Cu) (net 1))
 (segment (start 145.219 81.153) (end 143.3775 81.153) (width 0.25) (layer F.Cu) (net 1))
 (segment (start 142.171 82.3595) (end 142.171 93.6625) (width 0.25) (layer F.Cu) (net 1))
 (segment (start 143.3775 81.153) (end 142.171 82.3595) (width 0.25) (layer F.Cu) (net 1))
 (segment (start 145.219 81.153) (end 149.537 81.153) (width 0.25) (layer B.Cu) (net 1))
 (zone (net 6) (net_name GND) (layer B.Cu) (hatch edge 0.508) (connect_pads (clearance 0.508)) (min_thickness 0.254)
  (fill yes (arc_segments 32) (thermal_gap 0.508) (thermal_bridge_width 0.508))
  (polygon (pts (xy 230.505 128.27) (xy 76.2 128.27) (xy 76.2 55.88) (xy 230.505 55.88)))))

